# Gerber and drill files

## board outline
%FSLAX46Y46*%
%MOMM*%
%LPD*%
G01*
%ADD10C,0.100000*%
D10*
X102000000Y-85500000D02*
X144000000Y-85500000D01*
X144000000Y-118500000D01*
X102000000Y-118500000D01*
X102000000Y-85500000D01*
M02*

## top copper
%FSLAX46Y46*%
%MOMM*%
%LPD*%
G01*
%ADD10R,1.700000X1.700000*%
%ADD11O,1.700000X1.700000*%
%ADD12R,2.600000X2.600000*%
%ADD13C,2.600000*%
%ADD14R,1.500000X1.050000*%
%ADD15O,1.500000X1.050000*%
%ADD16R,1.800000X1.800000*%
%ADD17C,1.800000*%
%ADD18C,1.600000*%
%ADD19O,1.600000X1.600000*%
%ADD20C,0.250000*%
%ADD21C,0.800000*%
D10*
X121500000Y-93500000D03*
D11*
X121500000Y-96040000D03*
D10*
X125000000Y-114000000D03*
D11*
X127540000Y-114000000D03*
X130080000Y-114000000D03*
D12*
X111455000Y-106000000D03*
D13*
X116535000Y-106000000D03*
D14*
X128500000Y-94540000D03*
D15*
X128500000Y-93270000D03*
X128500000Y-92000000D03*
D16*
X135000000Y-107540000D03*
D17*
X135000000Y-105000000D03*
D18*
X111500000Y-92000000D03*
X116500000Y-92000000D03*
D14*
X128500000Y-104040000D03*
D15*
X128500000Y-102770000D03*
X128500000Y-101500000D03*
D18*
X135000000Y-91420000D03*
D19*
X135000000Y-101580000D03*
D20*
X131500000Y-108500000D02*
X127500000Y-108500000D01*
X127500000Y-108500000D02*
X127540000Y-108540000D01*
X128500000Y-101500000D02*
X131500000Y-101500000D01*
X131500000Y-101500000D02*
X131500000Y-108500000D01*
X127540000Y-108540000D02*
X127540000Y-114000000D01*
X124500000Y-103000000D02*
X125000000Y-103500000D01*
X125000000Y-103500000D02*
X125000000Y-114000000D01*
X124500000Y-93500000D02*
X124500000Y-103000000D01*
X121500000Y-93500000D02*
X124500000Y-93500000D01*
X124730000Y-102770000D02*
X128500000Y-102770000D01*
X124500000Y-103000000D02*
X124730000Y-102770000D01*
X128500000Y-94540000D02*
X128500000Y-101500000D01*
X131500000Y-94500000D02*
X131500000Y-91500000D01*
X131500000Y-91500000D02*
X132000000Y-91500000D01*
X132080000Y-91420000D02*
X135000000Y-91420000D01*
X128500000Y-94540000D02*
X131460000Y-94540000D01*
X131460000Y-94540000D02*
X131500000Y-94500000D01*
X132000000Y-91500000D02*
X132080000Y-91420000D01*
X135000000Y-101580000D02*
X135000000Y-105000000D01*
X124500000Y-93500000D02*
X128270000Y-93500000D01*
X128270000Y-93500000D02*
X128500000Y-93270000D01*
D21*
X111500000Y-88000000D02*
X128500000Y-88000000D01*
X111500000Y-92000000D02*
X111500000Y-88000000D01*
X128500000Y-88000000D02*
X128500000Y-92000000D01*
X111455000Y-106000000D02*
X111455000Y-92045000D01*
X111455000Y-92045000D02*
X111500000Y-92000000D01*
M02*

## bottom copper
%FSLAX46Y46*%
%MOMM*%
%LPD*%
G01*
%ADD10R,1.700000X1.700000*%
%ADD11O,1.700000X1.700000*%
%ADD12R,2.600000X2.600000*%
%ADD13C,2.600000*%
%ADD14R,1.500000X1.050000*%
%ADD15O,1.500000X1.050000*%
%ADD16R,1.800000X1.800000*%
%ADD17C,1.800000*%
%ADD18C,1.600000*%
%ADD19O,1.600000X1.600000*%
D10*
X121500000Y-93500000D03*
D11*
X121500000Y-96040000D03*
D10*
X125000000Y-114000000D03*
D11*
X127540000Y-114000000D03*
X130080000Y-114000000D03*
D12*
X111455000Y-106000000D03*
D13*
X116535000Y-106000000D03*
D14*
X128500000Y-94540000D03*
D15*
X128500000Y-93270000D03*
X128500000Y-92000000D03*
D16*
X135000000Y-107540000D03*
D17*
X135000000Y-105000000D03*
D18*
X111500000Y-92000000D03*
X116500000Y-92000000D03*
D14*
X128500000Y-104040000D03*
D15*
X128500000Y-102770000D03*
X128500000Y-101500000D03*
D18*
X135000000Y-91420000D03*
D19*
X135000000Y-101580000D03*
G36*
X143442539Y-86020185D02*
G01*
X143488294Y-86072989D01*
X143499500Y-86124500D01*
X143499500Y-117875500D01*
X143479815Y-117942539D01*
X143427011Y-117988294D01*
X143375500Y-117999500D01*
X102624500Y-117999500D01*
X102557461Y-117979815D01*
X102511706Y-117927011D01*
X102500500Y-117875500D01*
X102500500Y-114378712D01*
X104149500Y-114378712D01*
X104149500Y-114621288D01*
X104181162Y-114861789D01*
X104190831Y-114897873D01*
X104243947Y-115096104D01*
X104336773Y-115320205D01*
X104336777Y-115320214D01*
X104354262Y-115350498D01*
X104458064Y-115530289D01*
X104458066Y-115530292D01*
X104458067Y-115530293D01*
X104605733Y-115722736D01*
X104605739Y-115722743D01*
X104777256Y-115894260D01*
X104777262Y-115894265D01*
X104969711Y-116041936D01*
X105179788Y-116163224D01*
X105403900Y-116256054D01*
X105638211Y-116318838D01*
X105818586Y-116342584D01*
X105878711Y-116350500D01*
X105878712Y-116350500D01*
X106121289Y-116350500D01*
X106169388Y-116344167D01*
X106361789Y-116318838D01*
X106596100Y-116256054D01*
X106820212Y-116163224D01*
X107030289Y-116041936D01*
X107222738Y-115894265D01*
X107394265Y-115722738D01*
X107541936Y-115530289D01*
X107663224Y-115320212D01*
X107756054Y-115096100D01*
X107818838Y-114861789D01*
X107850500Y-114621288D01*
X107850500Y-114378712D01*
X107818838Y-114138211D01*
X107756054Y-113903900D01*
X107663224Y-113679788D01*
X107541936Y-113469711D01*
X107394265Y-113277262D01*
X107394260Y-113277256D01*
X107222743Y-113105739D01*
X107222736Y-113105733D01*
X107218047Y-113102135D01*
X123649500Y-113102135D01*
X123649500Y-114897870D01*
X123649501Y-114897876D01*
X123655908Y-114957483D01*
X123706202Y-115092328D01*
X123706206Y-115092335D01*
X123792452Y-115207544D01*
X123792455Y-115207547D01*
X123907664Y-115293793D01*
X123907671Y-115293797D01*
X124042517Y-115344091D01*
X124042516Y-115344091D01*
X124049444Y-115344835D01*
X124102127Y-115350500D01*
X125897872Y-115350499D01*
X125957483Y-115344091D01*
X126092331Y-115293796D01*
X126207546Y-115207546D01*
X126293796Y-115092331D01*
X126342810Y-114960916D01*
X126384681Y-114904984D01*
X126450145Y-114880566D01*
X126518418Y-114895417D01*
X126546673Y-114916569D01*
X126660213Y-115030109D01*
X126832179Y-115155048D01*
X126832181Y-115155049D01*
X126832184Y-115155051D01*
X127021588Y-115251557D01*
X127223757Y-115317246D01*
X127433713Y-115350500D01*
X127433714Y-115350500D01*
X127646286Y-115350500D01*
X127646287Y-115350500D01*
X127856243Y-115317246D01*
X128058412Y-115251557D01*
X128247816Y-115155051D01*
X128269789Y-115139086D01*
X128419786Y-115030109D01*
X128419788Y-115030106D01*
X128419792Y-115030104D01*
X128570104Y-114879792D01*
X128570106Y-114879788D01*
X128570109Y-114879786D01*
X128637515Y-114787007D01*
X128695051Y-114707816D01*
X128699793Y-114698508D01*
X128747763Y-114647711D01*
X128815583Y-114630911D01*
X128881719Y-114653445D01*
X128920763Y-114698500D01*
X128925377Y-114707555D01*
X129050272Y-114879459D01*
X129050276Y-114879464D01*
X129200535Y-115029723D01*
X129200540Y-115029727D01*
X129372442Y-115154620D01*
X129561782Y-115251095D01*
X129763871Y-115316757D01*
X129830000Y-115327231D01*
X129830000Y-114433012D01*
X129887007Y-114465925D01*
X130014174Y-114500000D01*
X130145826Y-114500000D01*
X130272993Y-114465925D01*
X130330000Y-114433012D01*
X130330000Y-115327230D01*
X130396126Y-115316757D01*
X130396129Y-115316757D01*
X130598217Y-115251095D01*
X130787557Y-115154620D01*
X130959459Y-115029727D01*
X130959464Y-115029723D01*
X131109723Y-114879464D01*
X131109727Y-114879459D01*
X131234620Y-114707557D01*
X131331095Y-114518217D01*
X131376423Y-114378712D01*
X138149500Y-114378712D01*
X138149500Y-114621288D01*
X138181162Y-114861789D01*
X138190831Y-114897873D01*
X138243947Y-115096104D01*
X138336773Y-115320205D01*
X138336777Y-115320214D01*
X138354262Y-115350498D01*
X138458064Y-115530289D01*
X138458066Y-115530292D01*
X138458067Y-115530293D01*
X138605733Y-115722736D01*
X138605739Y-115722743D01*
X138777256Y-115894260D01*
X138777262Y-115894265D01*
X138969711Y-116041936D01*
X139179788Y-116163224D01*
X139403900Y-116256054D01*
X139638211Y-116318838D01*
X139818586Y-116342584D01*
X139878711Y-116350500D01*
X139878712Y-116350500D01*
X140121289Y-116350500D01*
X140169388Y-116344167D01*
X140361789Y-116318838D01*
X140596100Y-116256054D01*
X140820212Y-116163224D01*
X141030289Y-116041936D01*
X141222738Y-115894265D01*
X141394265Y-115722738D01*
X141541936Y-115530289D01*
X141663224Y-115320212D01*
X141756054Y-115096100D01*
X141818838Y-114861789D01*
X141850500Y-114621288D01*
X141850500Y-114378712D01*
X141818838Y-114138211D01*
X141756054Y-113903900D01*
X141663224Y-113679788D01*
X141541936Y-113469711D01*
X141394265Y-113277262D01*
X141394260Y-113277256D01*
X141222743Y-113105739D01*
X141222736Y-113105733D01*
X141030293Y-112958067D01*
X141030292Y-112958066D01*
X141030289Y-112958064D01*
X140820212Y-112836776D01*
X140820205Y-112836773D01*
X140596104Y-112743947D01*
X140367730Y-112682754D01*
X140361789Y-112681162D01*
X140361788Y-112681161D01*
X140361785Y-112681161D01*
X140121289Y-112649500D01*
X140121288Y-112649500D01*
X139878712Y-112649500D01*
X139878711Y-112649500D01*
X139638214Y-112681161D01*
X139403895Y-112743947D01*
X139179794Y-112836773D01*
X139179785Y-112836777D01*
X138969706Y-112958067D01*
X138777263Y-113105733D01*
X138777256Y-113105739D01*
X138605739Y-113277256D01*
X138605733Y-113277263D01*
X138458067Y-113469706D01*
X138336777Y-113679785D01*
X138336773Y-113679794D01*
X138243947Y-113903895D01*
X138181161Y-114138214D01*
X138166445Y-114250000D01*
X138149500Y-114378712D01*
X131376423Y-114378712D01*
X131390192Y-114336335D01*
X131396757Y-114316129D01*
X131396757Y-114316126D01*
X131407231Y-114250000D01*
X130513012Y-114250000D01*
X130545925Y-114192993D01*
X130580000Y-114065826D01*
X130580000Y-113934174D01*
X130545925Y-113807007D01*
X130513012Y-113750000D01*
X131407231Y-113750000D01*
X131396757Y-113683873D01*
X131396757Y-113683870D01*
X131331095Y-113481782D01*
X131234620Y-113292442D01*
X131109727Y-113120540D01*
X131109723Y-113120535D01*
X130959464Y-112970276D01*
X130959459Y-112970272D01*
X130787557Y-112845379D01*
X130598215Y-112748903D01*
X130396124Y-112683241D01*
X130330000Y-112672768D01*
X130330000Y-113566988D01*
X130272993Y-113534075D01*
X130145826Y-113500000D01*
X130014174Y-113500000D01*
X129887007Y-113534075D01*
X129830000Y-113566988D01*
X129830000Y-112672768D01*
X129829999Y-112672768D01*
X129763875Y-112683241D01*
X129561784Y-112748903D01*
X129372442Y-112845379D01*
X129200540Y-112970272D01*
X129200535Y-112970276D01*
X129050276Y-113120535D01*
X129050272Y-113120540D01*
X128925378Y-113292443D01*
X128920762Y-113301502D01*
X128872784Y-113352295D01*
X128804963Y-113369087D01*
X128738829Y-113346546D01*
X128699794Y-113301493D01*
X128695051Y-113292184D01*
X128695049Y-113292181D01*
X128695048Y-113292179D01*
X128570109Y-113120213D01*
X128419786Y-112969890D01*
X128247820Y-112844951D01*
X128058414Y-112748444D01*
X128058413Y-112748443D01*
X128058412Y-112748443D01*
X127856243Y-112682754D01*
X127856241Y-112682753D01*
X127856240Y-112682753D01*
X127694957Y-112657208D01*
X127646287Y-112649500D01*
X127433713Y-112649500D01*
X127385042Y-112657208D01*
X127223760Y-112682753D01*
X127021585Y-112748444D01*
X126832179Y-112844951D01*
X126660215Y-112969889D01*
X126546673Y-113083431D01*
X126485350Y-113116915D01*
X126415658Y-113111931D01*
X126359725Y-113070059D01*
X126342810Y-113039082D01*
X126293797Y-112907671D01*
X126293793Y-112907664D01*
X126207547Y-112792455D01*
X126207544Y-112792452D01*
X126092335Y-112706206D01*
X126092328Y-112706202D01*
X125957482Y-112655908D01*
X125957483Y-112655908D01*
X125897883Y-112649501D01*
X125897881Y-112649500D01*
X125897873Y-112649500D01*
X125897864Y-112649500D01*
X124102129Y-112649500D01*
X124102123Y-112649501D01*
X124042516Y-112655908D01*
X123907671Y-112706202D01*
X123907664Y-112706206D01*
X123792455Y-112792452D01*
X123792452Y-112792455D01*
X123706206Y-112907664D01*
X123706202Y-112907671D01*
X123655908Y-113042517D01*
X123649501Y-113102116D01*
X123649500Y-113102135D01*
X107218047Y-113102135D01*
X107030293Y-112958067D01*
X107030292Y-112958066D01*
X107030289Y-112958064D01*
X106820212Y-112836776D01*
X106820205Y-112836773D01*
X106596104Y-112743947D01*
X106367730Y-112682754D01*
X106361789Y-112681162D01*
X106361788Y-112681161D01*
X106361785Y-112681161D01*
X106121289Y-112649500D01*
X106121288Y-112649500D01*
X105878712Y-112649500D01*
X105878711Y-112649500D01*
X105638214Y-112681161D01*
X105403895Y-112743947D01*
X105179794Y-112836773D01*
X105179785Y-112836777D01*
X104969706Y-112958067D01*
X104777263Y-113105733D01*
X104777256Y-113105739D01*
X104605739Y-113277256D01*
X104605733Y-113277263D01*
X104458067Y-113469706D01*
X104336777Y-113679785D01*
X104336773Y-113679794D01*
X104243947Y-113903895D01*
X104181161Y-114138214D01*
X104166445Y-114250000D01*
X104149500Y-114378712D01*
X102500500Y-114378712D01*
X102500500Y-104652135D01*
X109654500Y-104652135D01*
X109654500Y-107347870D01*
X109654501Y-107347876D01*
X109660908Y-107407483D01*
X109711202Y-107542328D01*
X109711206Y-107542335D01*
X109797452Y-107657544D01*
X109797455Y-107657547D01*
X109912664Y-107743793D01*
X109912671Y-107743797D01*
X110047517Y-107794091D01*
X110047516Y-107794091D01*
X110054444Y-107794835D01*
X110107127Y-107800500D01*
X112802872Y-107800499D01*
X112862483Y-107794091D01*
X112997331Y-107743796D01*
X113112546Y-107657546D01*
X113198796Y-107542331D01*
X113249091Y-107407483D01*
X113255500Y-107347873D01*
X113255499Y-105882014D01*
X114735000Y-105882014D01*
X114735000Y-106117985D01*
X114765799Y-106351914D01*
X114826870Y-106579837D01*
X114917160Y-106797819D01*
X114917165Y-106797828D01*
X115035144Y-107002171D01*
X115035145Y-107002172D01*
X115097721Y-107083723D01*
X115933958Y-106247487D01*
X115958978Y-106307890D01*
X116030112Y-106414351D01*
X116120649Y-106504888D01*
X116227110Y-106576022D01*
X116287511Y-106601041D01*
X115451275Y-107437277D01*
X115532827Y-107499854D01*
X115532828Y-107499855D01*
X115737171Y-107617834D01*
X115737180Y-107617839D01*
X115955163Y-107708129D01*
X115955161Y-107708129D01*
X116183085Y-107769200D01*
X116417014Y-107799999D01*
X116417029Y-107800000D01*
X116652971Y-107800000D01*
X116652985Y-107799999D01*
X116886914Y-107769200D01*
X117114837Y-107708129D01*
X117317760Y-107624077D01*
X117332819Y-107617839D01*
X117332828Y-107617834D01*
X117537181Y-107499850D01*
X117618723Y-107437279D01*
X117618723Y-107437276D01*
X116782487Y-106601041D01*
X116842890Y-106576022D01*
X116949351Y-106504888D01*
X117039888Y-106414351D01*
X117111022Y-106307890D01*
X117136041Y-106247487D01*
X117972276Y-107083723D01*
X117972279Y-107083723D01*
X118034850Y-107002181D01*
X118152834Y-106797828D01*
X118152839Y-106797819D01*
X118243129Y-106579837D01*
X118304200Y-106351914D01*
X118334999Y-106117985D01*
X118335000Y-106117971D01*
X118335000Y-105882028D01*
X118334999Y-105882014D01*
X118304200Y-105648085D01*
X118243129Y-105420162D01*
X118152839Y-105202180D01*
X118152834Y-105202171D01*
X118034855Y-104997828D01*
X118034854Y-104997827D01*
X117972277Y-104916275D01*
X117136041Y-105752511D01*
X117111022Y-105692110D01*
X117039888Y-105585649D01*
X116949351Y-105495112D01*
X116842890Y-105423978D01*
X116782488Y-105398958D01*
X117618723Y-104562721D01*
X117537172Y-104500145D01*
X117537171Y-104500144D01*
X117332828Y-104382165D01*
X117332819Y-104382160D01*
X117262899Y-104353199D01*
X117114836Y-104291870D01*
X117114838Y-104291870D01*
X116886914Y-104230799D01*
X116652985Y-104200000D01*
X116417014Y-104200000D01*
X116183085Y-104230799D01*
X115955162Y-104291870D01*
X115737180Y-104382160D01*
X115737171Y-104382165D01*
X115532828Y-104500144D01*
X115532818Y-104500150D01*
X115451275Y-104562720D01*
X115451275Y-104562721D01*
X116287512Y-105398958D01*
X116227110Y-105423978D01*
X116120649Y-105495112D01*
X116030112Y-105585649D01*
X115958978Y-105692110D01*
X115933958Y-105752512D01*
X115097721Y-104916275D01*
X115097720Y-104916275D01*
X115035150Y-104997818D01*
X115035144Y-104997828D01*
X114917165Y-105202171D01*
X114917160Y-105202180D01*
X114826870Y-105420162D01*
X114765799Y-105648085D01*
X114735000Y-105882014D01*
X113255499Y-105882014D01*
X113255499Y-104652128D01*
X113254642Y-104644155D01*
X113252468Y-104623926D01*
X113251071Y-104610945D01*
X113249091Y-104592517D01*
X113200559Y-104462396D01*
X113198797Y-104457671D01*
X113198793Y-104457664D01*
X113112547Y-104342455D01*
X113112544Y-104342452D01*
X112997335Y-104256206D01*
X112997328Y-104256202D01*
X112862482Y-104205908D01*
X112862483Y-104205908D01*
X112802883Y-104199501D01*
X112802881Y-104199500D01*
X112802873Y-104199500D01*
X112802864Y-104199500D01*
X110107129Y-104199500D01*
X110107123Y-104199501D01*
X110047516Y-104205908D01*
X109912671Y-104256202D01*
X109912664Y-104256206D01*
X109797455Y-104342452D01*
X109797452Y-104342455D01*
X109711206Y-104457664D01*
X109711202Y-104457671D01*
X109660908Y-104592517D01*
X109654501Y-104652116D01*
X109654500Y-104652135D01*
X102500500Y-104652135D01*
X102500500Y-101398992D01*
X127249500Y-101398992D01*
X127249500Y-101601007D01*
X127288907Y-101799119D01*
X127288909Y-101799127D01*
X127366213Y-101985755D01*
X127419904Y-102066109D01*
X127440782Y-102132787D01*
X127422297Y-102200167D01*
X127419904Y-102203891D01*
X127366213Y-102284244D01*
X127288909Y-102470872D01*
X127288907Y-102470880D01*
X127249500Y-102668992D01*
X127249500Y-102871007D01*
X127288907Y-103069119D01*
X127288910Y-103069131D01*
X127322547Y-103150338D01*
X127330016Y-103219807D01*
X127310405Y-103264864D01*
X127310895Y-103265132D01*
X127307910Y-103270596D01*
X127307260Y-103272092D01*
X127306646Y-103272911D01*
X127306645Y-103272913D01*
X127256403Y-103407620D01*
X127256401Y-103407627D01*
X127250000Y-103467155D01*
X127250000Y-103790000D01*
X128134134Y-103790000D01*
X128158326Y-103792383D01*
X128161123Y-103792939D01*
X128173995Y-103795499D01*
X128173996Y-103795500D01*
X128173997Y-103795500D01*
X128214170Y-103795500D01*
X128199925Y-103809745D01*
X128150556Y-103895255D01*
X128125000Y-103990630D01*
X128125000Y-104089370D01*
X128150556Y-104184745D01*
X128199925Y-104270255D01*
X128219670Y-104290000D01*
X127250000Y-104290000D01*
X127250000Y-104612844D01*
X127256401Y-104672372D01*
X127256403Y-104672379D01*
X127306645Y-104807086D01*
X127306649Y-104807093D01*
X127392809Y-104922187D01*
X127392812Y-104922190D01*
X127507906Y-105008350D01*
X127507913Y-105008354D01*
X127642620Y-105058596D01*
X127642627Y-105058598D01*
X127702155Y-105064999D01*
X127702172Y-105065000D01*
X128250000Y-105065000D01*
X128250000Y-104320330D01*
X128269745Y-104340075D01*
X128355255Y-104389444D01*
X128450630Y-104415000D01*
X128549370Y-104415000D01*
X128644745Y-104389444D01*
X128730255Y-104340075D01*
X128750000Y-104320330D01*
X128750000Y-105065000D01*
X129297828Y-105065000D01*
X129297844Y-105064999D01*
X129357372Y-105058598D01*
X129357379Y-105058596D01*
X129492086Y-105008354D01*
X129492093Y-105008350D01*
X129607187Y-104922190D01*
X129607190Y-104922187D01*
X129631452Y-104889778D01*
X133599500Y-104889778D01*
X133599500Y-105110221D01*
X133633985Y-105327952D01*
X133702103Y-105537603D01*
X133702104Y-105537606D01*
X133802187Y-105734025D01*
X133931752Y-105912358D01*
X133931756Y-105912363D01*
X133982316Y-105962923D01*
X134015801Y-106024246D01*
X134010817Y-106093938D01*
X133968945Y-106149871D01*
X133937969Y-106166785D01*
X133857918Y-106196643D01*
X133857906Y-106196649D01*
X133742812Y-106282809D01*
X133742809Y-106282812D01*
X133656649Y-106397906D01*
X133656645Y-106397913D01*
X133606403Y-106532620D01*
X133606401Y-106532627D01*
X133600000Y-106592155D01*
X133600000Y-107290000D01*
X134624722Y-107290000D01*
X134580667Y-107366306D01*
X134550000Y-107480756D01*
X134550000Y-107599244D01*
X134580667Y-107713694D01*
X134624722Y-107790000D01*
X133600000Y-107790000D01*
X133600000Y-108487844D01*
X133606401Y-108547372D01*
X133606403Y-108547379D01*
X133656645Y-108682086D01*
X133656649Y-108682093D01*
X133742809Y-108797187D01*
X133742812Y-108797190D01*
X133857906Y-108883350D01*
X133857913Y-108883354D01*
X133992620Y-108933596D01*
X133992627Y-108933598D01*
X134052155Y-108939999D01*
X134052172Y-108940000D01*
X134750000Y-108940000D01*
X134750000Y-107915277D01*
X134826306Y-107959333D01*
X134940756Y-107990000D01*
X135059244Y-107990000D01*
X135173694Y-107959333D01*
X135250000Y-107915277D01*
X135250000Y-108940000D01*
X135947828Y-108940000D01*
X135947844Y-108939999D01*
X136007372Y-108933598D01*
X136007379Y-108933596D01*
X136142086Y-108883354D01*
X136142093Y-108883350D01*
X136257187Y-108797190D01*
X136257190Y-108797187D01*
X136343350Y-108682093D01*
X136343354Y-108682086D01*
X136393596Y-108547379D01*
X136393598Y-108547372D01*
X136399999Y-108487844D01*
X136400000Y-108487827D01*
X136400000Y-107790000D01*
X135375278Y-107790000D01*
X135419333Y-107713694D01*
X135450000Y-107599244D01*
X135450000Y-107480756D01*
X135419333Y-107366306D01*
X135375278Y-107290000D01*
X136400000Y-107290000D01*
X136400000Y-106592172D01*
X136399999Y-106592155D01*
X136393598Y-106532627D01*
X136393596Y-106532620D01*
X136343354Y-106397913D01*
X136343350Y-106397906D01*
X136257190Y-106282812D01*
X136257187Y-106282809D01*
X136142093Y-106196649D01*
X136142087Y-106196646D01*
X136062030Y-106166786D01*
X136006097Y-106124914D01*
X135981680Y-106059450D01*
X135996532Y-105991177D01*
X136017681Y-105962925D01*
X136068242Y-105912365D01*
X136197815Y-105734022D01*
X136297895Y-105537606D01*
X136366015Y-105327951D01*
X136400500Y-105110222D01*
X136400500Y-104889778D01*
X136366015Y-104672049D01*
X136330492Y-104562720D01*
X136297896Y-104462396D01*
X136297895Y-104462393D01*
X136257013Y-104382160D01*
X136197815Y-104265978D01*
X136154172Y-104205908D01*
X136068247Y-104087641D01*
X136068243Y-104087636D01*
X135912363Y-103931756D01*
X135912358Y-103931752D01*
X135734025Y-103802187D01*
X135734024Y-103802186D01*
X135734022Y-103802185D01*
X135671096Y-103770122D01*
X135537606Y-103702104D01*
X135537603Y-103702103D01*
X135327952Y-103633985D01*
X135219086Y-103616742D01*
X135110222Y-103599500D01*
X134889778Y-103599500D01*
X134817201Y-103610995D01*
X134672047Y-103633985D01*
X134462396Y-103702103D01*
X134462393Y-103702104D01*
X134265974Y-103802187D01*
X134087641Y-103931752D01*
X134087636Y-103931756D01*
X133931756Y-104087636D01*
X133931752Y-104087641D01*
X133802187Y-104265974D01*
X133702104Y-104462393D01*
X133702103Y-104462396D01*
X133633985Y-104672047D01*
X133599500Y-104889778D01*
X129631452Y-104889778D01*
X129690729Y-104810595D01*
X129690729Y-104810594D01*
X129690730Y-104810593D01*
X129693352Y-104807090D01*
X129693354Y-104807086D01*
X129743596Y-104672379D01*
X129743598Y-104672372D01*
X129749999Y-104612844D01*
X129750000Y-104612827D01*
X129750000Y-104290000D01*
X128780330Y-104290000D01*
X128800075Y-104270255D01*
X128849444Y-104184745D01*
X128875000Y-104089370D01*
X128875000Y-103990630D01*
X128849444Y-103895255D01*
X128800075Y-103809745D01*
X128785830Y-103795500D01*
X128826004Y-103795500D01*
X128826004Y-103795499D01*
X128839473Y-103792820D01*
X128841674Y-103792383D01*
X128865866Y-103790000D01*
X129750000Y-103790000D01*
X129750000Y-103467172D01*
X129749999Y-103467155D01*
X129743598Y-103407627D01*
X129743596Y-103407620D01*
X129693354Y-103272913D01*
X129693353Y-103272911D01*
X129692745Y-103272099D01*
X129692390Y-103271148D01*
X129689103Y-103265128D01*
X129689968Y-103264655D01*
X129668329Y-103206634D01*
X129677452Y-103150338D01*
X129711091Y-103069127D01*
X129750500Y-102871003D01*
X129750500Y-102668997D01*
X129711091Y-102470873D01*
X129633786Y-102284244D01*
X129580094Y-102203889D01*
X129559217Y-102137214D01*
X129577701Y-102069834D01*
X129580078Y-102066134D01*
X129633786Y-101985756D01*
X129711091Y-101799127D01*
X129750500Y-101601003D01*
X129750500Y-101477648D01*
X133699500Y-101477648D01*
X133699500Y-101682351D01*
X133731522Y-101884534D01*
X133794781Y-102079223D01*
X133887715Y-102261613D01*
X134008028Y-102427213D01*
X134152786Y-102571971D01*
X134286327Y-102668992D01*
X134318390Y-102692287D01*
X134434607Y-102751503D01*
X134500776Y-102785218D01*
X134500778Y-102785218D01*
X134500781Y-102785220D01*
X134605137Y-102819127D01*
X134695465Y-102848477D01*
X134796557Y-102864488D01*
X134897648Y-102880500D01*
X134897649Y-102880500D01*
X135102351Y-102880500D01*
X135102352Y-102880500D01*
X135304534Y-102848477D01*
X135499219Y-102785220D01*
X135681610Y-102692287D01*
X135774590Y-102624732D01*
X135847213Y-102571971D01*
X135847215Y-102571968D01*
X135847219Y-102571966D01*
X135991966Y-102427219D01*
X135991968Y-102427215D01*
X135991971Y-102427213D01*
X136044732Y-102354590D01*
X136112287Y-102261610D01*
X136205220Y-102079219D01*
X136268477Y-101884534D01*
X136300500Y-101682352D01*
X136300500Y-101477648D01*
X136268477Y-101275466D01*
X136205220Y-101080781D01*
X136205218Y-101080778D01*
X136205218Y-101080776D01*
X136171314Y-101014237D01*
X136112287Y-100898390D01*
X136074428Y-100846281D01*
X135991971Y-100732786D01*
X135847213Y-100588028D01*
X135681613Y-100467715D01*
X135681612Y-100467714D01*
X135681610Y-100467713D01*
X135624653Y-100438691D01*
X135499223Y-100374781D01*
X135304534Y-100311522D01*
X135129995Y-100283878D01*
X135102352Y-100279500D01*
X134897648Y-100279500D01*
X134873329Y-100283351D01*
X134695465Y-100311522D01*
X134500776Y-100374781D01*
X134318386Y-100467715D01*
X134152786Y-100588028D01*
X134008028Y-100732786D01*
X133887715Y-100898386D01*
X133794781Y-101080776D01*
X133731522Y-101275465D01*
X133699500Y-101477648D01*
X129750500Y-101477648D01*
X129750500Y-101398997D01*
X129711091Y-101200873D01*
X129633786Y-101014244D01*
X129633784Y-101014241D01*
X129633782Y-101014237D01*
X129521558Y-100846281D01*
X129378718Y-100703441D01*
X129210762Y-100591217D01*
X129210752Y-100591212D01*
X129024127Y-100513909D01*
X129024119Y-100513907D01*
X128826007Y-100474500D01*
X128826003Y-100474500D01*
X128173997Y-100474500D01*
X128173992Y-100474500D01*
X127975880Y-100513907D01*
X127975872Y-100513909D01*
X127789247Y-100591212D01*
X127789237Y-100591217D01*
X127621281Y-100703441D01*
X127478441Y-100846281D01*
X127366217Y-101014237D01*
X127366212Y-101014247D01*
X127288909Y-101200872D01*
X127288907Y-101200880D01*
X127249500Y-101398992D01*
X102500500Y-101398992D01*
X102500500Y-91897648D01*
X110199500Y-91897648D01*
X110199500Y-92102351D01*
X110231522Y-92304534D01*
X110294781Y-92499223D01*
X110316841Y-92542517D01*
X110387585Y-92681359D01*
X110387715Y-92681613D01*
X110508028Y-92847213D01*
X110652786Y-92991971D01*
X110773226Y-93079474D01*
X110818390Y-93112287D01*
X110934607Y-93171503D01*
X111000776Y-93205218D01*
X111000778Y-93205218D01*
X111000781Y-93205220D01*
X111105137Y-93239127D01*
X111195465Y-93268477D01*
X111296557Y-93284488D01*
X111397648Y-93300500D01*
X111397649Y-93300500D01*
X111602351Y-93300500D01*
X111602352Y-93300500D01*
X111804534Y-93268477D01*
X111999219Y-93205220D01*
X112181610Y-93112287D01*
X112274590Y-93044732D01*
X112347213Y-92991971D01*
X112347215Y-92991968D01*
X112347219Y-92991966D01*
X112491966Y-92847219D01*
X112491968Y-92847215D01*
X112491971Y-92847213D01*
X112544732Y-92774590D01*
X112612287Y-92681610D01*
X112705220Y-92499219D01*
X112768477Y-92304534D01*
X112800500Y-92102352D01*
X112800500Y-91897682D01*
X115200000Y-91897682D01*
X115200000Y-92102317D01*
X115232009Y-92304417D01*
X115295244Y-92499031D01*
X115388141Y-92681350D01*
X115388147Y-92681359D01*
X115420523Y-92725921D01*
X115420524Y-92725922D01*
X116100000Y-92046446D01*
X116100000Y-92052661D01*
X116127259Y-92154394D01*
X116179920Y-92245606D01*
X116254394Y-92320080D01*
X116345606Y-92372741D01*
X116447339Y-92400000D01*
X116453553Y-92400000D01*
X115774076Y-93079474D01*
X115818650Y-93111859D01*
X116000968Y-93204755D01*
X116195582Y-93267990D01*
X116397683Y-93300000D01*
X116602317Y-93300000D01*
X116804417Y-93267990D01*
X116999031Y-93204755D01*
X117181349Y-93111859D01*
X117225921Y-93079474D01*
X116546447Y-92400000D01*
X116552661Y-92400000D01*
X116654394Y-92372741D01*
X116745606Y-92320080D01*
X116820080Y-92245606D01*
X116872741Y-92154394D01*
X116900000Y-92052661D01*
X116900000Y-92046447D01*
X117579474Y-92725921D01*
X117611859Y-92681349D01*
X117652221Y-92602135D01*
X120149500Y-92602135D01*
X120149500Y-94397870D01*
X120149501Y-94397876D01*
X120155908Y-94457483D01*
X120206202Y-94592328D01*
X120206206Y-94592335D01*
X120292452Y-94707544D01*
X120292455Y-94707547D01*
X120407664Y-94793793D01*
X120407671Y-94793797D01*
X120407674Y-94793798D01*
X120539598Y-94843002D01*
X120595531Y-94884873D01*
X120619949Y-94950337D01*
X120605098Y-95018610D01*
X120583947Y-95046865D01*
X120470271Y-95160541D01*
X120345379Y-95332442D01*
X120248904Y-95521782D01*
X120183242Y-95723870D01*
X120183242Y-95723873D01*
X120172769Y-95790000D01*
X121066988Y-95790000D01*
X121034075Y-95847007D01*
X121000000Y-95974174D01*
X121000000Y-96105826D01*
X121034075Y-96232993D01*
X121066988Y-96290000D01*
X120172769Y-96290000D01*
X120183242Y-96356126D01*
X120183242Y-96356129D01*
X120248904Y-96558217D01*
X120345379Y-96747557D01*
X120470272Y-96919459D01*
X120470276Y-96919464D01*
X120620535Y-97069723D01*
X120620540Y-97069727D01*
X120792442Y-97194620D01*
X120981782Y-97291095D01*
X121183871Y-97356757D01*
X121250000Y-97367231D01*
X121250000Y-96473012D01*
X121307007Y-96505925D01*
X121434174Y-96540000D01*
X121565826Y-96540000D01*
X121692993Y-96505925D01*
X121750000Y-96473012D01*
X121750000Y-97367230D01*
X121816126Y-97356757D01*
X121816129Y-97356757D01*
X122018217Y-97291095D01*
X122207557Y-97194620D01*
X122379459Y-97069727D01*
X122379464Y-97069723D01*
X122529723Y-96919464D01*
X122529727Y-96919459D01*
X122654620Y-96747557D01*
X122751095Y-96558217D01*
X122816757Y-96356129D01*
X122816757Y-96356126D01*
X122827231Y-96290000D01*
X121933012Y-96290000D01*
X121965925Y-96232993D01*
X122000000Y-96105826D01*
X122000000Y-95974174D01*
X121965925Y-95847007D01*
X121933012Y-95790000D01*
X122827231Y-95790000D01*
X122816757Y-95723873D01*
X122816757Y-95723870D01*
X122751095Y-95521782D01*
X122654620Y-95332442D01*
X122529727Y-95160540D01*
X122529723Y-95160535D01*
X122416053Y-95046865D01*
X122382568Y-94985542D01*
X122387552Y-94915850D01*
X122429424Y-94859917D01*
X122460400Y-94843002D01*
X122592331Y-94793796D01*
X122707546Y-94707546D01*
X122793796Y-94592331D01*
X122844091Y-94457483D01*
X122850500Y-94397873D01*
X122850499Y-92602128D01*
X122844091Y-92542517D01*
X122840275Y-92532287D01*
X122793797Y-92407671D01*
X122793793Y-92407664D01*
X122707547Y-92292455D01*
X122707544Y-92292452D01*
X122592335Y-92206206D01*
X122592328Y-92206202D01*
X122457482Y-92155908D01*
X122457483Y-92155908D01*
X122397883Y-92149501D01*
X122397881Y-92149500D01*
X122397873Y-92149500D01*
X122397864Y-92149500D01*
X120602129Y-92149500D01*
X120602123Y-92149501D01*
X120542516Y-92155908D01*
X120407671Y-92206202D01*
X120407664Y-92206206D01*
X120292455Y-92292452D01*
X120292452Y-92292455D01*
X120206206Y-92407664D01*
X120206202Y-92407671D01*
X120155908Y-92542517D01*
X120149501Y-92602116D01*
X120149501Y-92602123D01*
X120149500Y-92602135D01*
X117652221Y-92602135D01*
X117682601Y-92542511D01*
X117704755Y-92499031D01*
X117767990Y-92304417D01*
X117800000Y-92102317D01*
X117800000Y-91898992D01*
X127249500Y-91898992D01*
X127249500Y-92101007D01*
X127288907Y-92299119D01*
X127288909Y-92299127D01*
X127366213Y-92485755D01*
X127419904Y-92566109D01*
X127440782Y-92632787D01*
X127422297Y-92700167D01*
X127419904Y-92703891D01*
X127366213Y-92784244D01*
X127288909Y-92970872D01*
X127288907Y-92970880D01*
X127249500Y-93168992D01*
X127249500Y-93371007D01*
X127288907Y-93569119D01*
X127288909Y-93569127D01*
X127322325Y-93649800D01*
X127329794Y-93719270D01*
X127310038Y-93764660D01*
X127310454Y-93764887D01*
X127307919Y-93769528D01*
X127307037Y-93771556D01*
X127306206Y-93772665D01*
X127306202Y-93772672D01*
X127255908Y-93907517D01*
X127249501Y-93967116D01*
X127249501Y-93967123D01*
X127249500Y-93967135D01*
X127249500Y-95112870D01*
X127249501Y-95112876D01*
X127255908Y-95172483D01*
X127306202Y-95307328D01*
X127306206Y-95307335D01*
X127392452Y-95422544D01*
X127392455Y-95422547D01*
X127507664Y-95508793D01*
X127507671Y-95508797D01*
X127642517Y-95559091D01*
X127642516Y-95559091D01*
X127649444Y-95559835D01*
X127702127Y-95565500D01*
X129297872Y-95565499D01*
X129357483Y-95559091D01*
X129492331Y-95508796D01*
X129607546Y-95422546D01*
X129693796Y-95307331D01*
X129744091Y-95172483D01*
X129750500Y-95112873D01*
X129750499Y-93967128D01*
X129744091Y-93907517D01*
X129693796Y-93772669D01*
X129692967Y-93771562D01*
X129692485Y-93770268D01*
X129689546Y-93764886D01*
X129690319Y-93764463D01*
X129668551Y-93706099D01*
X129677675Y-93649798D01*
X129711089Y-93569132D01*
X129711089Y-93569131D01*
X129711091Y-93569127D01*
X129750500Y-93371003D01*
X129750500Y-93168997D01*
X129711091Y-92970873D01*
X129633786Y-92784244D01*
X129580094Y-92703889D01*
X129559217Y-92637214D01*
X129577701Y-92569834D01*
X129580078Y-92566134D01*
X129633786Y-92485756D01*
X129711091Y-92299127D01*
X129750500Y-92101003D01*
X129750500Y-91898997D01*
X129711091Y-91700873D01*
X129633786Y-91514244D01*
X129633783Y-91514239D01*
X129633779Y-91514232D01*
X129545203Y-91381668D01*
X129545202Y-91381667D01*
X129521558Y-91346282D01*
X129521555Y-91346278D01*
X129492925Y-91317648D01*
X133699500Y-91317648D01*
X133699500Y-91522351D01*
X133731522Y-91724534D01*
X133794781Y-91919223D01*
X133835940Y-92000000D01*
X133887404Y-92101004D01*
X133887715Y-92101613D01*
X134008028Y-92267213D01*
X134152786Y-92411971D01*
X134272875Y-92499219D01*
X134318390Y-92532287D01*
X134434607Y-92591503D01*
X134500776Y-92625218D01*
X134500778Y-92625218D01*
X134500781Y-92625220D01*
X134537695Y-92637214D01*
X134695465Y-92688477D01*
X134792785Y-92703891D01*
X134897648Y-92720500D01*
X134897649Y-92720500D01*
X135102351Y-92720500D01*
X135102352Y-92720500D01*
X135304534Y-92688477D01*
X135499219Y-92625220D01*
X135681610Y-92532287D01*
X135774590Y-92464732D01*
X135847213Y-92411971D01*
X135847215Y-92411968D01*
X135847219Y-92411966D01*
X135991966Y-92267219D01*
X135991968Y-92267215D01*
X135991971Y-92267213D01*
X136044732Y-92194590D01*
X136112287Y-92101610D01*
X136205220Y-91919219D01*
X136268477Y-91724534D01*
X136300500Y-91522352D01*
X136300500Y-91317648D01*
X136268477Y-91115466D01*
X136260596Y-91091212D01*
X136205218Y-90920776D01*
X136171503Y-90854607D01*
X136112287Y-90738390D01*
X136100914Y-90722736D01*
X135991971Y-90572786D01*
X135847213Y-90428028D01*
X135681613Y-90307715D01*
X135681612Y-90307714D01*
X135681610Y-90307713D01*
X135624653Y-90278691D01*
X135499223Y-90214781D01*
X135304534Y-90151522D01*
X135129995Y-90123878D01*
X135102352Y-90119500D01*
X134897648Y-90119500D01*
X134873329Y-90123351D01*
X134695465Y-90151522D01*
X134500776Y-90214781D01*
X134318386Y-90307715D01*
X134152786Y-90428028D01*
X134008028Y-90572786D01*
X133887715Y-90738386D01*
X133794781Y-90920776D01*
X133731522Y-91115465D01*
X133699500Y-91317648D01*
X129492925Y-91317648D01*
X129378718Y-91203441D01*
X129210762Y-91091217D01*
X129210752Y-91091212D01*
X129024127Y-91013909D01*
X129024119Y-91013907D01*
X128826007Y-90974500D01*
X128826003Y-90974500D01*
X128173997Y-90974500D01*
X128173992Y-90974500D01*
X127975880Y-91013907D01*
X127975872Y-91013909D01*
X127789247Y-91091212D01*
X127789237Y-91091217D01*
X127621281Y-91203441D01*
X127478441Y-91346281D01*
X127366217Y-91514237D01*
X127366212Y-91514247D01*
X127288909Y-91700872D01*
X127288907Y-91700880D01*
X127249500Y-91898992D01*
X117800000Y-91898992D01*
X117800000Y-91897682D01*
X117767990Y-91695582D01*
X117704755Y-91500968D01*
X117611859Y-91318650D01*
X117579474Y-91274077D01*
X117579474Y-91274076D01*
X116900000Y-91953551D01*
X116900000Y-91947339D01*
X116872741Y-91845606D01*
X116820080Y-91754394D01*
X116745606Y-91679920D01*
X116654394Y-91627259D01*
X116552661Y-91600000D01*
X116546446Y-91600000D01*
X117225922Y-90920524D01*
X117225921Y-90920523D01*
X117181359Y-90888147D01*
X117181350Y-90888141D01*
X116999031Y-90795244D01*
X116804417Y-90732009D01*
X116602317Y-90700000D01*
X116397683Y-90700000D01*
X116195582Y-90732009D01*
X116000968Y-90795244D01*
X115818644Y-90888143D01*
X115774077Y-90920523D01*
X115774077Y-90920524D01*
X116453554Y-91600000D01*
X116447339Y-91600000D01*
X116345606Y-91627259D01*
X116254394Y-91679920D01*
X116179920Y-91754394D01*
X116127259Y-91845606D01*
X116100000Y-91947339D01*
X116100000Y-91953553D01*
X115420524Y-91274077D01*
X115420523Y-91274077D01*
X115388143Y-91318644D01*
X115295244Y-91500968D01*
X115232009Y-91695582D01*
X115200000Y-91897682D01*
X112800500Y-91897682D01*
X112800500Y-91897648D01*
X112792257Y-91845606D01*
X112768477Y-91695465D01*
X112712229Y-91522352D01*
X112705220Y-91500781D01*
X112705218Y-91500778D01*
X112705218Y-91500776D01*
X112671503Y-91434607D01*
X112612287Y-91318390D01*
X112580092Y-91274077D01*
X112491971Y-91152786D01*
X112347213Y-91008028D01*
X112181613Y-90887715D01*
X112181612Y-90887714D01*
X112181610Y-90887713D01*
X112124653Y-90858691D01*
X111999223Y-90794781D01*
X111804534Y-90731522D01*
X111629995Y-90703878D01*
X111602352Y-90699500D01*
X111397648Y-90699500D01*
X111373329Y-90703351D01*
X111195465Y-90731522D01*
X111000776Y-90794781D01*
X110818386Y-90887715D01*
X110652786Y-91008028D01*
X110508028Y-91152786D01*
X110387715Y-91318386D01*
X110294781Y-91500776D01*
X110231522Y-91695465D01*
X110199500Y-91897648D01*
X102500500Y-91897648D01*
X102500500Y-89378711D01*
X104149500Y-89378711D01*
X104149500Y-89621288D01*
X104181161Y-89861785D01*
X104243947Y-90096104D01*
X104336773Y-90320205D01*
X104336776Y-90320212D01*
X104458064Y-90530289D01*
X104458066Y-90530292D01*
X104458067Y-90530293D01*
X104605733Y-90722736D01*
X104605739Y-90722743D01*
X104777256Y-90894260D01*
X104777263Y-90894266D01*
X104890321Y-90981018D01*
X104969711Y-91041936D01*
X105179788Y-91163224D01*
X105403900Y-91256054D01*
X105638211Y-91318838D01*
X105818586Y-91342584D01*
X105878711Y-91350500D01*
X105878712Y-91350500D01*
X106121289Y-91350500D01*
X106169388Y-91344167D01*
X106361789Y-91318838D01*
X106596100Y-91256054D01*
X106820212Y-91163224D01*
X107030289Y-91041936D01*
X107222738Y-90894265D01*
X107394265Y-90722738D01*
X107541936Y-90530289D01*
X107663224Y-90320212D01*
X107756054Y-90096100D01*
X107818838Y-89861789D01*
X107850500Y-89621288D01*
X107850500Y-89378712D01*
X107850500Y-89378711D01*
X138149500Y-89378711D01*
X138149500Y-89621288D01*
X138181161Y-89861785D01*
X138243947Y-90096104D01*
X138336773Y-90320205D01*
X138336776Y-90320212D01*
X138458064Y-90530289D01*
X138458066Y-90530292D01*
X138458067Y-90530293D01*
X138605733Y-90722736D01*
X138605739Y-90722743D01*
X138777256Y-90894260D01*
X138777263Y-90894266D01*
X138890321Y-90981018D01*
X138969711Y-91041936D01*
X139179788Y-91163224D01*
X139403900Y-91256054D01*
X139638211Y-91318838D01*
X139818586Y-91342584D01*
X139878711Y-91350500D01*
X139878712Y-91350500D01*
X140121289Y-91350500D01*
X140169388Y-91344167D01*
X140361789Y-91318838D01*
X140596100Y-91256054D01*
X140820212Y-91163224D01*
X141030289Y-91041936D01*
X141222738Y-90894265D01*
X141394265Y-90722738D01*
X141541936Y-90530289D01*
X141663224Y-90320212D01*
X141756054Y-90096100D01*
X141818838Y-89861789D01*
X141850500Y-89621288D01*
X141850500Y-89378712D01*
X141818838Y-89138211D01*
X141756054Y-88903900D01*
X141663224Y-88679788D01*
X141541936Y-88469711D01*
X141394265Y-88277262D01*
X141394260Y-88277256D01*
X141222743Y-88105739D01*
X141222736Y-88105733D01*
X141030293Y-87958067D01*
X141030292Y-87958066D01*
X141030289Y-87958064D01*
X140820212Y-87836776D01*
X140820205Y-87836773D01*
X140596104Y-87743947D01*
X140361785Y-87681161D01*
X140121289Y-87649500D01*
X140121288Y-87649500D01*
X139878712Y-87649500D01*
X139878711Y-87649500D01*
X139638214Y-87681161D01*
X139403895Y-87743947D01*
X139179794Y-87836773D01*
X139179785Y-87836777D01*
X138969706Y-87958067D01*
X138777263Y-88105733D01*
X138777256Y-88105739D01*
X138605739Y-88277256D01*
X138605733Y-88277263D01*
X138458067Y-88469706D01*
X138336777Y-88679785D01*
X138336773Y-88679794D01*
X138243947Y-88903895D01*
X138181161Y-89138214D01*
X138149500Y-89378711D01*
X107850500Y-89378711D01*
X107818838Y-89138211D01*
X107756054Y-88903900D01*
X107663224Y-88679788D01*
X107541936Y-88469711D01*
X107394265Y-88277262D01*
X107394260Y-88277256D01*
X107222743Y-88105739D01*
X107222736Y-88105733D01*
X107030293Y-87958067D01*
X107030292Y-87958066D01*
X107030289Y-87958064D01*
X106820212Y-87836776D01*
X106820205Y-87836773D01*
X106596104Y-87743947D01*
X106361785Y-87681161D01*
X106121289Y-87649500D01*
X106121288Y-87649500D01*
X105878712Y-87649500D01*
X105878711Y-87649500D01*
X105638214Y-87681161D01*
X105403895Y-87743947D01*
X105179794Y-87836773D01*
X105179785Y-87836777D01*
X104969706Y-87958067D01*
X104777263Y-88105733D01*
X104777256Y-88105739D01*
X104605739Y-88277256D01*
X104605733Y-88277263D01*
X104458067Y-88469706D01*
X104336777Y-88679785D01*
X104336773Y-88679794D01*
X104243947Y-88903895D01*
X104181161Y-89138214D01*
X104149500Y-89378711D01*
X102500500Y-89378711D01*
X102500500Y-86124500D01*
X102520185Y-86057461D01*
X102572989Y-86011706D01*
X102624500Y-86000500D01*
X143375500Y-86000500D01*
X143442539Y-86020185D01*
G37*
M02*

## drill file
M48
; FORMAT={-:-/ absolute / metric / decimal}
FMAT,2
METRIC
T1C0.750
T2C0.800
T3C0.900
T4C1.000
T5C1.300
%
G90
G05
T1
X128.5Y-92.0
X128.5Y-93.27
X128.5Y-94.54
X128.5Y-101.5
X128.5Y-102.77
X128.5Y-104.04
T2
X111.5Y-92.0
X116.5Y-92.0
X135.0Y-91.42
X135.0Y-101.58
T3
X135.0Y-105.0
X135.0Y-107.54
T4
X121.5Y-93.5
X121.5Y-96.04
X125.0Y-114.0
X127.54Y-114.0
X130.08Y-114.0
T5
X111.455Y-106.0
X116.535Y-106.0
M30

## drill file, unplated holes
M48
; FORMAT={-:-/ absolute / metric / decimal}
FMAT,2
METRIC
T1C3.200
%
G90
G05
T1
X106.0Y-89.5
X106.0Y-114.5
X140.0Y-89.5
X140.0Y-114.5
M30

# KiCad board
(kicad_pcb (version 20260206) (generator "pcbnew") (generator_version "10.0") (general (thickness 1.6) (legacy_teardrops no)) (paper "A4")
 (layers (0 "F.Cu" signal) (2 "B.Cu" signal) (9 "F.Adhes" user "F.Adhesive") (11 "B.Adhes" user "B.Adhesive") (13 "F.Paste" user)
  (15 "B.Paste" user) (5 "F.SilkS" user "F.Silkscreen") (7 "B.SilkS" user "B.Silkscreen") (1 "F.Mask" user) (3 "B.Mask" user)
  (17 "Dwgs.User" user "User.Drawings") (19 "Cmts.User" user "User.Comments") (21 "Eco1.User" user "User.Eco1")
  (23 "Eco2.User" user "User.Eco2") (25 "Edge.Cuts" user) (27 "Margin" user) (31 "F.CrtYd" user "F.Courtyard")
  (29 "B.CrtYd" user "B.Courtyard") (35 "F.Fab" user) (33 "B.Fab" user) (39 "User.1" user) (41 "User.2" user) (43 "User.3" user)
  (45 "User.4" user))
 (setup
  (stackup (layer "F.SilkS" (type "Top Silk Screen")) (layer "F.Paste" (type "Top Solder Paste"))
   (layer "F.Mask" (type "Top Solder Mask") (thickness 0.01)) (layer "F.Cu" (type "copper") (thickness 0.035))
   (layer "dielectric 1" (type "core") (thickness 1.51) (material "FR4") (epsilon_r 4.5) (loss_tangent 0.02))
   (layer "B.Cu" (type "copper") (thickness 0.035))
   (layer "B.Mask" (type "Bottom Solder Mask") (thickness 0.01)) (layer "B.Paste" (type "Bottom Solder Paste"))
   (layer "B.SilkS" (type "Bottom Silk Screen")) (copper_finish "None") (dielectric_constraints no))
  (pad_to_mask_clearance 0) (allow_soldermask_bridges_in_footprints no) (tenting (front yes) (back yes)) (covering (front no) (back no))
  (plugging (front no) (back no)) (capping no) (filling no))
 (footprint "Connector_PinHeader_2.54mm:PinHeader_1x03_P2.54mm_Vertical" (layer "F.Cu") (at 125 114 90)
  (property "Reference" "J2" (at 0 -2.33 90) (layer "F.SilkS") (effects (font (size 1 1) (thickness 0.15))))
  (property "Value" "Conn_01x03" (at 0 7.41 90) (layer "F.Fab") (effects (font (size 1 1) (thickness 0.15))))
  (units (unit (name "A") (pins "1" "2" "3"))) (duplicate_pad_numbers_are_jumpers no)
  (pad "1" thru_hole rect (at 0 0 90) (size 1.7 1.7) (drill 1) (layers "*.Cu" "*.Mask") (remove_unused_layers no) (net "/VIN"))
  (pad "2" thru_hole oval (at 0 2.54 90) (size 1.7 1.7) (drill 1) (layers "*.Cu" "*.Mask") (remove_unused_layers no) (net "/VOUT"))
  (pad "3" thru_hole oval (at 0 5.08 90) (size 1.7 1.7) (drill 1) (layers "*.Cu" "*.Mask") (remove_unused_layers no) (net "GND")))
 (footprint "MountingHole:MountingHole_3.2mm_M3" (layer "F.Cu") (at 140 89.5)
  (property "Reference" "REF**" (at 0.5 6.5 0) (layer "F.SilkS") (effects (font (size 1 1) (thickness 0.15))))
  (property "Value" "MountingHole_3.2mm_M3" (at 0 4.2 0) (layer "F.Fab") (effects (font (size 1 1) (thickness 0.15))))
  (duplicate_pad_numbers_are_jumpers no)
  (pad "" np_thru_hole circle (at 0 0) (size 3.2 3.2) (drill 3.2) (layers "*.Cu" "*.Mask")))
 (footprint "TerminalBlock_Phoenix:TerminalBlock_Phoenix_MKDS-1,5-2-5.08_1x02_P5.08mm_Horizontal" (layer "F.Cu") (at 111.455 106)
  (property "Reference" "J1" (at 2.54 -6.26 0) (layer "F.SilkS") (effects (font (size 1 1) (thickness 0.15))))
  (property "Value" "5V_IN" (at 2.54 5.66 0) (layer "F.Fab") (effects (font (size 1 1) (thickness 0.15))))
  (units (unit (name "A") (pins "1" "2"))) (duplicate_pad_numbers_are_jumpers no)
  (pad "1" thru_hole rect (at 0 0) (size 2.6 2.6) (drill 1.3) (layers "*.Cu" "*.Mask") (remove_unused_layers no) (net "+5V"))
  (pad "2" thru_hole circle (at 5.08 0) (size 2.6 2.6) (drill 1.3) (layers "*.Cu" "*.Mask") (remove_unused_layers no) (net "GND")))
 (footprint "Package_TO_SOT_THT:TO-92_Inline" (layer "F.Cu") (at 128.5 94.54 90)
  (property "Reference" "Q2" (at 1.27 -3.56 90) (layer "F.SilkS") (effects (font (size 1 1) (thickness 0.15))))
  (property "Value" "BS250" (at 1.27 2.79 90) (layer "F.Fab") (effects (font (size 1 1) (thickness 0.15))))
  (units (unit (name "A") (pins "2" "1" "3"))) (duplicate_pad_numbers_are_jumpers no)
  (pad "1" thru_hole rect (at 0 0 90) (size 1.05 1.5) (drill 0.75) (layers "*.Cu" "*.Mask") (remove_unused_layers no) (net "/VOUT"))
  (pad "2" thru_hole oval (at 1.27 0 90) (size 1.05 1.5) (drill 0.75) (layers "*.Cu" "*.Mask") (remove_unused_layers no) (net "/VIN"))
  (pad "3" thru_hole oval (at 2.54 0 90) (size 1.05 1.5) (drill 0.75) (layers "*.Cu" "*.Mask") (remove_unused_layers no) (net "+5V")))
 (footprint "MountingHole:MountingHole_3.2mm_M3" (layer "F.Cu") (at 106 89.5)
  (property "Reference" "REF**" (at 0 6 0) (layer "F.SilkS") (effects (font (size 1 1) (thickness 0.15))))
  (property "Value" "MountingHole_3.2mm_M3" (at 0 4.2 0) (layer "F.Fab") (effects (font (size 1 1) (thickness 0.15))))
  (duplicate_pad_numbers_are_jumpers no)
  (pad "" np_thru_hole circle (at 0 0) (size 3.2 3.2) (drill 3.2) (layers "*.Cu" "*.Mask")))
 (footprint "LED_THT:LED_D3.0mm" (layer "F.Cu") (at 135 107.54 90)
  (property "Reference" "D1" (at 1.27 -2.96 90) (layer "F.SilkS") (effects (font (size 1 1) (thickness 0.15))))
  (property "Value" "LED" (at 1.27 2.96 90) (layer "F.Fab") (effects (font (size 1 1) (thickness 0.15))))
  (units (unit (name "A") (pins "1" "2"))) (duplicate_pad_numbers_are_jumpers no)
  (pad "1" thru_hole rect (at 0 0 90) (size 1.8 1.8) (drill 0.9) (layers "*.Cu" "*.Mask") (remove_unused_layers no) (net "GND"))
  (pad "2" thru_hole circle (at 2.54 0 90) (size 1.8 1.8) (drill 0.9) (layers "*.Cu" "*.Mask") (remove_unused_layers no) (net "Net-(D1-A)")))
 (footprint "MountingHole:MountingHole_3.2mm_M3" (layer "F.Cu") (at 106 114.5)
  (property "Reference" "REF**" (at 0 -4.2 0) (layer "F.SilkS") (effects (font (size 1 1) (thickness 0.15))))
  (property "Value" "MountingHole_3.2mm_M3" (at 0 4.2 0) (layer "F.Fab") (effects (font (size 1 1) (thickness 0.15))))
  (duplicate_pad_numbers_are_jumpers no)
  (pad "" np_thru_hole circle (at 0 0) (size 3.2 3.2) (drill 3.2) (layers "*.Cu" "*.Mask")))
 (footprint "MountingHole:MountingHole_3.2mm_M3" (layer "F.Cu") (at 140 114.5)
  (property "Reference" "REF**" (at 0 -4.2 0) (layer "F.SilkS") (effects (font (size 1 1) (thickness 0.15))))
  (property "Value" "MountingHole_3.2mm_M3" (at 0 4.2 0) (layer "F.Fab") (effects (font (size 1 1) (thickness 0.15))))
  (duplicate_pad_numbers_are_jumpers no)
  (pad "" np_thru_hole circle (at 0 0) (size 3.2 3.2) (drill 3.2) (layers "*.Cu" "*.Mask")))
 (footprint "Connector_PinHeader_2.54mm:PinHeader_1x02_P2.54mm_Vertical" (layer "F.Cu") (at 121.5 93.5)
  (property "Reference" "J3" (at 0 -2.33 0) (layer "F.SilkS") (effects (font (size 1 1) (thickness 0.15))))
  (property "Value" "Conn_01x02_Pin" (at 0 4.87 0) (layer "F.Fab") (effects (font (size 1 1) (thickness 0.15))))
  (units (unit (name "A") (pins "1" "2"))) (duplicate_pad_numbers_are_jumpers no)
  (pad "1" thru_hole rect (at 0 0) (size 1.7 1.7) (drill 1) (layers "*.Cu" "*.Mask") (remove_unused_layers no) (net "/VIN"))
  (pad "2" thru_hole oval (at 0 2.54) (size 1.7 1.7) (drill 1) (layers "*.Cu" "*.Mask") (remove_unused_layers no) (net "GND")))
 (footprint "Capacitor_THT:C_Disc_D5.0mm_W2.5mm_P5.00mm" (layer "F.Cu") (at 111.5 92)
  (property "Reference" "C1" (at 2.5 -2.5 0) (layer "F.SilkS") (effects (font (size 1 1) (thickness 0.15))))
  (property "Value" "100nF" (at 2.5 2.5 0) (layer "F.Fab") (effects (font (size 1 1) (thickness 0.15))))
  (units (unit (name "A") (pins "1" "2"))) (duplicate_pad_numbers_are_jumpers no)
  (pad "1" thru_hole circle (at 0 0) (size 1.6 1.6) (drill 0.8) (layers "*.Cu" "*.Mask") (remove_unused_layers no) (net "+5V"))
  (pad "2" thru_hole circle (at 5 0) (size 1.6 1.6) (drill 0.8) (layers "*.Cu" "*.Mask") (remove_unused_layers no) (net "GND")))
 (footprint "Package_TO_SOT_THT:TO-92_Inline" (layer "F.Cu") (at 128.5 104.04 90)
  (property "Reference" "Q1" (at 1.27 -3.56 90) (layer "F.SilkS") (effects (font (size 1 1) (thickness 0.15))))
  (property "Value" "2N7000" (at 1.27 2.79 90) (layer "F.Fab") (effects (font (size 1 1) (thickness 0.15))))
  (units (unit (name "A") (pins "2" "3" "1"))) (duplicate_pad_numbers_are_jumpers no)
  (pad "1" thru_hole rect (at 0 0 90) (size 1.05 1.5) (drill 0.75) (layers "*.Cu" "*.Mask") (remove_unused_layers no) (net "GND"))
  (pad "2" thru_hole oval (at 1.27 0 90) (size 1.05 1.5) (drill 0.75) (layers "*.Cu" "*.Mask") (remove_unused_layers no) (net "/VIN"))
  (pad "3" thru_hole oval (at 2.54 0 90) (size 1.05 1.5) (drill 0.75) (layers "*.Cu" "*.Mask") (remove_unused_layers no) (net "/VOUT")))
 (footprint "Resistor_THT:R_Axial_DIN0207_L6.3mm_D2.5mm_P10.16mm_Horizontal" (layer "F.Cu") (at 135 91.42 -90)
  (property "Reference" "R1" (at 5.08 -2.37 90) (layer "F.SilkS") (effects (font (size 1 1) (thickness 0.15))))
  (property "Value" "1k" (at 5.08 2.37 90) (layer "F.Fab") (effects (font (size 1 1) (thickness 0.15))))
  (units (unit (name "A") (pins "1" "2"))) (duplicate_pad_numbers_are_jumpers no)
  (pad "1" thru_hole circle (at 0 0 270) (size 1.6 1.6) (drill 0.8) (layers "*.Cu" "*.Mask") (remove_unused_layers no) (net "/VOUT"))
  (pad "2" thru_hole oval (at 10.16 0 270) (size 1.6 1.6) (drill 0.8) (layers "*.Cu" "*.Mask") (remove_unused_layers no) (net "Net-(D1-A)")))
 (gr_rect (start 102 85.5) (end 144 118.5) (stroke (width 0.1) (type solid)) (fill no) (layer "Edge.Cuts"))
 (segment (start 121.5 93.5) (end 124.5 93.5) (width 0.25) (layer "F.Cu") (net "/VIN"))
 (segment (start 124.5 103) (end 125 103.5) (width 0.25) (layer "F.Cu") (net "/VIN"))
 (segment (start 124.5 103) (end 124.73 102.77) (width 0.25) (layer "F.Cu") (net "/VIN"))
 (segment (start 128.27 93.5) (end 128.5 93.27) (width 0.25) (layer "F.Cu") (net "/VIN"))
 (segment (start 124.73 102.77) (end 128.5 102.77) (width 0.25) (layer "F.Cu") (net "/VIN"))
 (segment (start 124.5 93.5) (end 124.5 103) (width 0.25) (layer "F.Cu") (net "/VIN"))
 (segment (start 124.5 93.5) (end 128.27 93.5) (width 0.25) (layer "F.Cu") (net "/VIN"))
 (segment (start 125 103.5) (end 125 114) (width 0.25) (layer "F.Cu") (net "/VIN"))
 (segment (start 128.5 94.54) (end 128.5 101.5) (width 0.25) (layer "F.Cu") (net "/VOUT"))
 (segment (start 131.5 91.5) (end 132 91.5) (width 0.25) (layer "F.Cu") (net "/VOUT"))
 (segment (start 127.54 108.54) (end 127.54 114) (width 0.25) (layer "F.Cu") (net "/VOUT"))
 (segment (start 132.08 91.42) (end 135 91.42) (width 0.25) (layer "F.Cu") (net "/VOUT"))
 (segment (start 131.5 94.5) (end 131.5 91.5) (width 0.25) (layer "F.Cu") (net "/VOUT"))
 (segment (start 131.5 101.5) (end 131.5 108.5) (width 0.25) (layer "F.Cu") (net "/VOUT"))
 (segment (start 131.46 94.54) (end 131.5 94.5) (width 0.25) (layer "F.Cu") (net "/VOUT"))
 (segment (start 127.5 108.5) (end 127.54 108.54) (width 0.25) (layer "F.Cu") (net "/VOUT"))
 (segment (start 131.5 108.5) (end 127.5 108.5) (width 0.25) (layer "F.Cu") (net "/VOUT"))
 (segment (start 128.5 94.54) (end 131.46 94.54) (width 0.25) (layer "F.Cu") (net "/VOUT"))
 (segment (start 128.5 101.5) (end 131.5 101.5) (width 0.25) (layer "F.Cu") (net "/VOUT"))
 (segment (start 132 91.5) (end 132.08 91.42) (width 0.25) (layer "F.Cu") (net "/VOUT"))
 (segment (start 111.455 92.045) (end 111.5 92) (width 0.8) (layer "F.Cu") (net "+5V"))
 (segment (start 111.5 88) (end 128.5 88) (width 0.8) (layer "F.Cu") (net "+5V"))
 (segment (start 111.455 106) (end 111.455 92.045) (width 0.8) (layer "F.Cu") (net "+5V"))
 (segment (start 128.5 88) (end 128.5 92) (width 0.8) (layer "F.Cu") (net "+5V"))
 (segment (start 111.5 92) (end 111.5 88) (width 0.8) (layer "F.Cu") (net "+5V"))
 (segment (start 135 101.58) (end 135 105) (width 0.25) (layer "F.Cu") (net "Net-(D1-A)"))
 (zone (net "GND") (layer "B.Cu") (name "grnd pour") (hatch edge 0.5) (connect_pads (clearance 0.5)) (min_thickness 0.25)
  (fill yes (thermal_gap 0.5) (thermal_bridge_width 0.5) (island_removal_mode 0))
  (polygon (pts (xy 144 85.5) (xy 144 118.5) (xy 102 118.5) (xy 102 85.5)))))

